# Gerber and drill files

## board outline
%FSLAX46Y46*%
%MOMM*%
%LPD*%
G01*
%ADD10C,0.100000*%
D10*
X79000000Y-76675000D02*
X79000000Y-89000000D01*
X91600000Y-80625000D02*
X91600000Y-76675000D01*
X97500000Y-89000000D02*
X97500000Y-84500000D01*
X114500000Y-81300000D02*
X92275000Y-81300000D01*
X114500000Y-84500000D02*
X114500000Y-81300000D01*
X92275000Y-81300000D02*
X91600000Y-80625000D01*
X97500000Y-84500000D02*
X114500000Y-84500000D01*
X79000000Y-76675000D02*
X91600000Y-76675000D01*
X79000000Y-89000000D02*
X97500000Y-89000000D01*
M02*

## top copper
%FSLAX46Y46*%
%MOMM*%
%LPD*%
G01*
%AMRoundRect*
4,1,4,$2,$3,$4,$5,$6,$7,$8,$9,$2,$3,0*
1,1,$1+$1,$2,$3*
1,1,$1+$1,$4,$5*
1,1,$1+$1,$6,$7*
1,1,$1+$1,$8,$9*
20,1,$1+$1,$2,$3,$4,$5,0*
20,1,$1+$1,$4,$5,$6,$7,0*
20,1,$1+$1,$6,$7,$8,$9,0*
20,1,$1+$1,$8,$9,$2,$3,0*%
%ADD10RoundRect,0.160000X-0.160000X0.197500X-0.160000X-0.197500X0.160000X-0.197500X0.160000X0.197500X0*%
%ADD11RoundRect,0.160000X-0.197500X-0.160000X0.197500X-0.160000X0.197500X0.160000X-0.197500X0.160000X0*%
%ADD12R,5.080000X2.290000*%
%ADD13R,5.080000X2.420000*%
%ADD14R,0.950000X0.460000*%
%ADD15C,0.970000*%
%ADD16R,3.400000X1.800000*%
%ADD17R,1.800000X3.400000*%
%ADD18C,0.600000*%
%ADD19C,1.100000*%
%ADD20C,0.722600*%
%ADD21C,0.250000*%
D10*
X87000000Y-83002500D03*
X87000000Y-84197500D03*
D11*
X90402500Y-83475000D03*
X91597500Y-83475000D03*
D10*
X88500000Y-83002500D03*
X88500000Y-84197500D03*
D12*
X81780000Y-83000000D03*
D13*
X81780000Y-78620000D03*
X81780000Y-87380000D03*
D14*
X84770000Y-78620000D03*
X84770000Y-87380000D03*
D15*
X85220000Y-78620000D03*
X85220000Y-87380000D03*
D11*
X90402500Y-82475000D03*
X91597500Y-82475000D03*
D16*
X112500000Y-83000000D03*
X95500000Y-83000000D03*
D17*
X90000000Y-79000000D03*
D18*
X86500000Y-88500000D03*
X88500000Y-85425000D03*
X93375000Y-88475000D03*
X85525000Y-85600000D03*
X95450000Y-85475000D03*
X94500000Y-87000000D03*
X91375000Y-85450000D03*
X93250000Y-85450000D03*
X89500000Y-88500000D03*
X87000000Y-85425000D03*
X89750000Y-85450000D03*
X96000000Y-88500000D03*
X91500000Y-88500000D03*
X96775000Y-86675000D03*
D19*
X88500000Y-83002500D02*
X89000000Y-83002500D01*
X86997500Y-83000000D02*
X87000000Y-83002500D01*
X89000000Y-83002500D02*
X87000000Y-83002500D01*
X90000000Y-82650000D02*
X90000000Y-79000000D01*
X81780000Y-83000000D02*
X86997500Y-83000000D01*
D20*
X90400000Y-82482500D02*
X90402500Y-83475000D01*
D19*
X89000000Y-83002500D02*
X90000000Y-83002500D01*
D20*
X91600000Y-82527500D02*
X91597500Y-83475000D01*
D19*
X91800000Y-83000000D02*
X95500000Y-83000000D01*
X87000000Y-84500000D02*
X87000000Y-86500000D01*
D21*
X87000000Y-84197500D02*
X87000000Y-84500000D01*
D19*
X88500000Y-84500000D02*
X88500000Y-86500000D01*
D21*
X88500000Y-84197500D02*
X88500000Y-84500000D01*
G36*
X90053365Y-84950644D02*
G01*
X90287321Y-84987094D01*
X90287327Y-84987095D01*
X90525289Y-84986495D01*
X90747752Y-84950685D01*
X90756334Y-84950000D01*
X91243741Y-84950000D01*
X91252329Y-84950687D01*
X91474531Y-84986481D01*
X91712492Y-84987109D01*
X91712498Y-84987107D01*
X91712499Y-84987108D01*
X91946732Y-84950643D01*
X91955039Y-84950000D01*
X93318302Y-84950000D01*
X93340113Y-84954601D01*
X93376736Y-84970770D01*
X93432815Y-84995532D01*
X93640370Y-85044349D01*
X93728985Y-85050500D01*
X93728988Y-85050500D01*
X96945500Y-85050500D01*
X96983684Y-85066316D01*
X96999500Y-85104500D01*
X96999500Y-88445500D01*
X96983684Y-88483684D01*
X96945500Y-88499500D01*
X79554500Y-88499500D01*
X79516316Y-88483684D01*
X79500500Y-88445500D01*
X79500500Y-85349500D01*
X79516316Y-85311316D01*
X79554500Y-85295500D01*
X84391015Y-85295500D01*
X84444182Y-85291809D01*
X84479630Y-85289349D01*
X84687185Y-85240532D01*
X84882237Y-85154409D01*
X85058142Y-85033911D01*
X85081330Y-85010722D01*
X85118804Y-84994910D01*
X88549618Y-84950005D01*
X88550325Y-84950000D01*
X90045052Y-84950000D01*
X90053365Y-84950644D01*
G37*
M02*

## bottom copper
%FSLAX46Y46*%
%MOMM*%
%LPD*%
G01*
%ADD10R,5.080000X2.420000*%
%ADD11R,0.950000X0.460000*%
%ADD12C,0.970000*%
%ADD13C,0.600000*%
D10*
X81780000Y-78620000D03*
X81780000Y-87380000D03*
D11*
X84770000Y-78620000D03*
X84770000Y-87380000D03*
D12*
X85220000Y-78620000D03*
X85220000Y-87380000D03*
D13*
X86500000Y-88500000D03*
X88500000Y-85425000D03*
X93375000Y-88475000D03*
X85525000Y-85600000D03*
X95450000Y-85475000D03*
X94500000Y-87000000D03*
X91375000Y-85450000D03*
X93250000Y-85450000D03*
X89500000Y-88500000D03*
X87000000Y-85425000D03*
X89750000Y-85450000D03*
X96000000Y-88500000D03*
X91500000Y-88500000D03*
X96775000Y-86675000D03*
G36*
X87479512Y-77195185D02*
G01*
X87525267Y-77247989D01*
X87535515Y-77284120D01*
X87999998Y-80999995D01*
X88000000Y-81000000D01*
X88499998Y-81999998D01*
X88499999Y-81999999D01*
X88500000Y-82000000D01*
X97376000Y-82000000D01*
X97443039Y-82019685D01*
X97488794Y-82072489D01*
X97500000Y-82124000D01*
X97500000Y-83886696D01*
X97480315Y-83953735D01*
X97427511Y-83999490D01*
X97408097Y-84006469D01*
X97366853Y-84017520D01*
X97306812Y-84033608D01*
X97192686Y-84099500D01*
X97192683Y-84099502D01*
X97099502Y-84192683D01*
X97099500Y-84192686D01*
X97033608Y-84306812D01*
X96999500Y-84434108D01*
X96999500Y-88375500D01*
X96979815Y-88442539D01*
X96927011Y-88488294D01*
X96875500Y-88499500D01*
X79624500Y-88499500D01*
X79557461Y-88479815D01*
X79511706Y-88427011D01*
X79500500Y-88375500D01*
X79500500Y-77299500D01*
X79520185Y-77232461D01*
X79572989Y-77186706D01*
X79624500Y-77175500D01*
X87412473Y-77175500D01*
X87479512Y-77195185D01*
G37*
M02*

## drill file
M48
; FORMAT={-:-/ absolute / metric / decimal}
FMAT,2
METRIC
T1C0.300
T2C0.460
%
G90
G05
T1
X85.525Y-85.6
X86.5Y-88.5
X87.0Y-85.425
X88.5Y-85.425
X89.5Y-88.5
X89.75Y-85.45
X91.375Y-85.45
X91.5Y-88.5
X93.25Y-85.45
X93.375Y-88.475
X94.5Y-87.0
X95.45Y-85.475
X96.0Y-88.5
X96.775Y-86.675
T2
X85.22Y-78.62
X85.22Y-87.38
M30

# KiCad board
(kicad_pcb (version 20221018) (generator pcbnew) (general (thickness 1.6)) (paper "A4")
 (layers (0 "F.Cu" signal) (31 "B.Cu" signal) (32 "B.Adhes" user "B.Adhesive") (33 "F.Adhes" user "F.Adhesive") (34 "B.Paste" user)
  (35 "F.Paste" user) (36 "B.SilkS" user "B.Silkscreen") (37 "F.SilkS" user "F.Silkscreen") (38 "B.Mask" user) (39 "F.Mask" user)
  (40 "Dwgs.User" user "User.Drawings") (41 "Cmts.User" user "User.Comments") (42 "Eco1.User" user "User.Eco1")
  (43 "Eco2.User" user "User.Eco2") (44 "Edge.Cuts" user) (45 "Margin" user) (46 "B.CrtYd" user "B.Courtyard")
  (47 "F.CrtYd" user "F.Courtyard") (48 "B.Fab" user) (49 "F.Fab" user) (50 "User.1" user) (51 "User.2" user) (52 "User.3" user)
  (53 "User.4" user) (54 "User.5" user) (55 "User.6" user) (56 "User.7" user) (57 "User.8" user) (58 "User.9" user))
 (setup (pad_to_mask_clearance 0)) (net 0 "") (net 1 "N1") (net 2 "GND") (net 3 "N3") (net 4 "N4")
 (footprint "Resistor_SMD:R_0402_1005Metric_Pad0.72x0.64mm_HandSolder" (layer "F.Cu") (at 87 83.6 -90)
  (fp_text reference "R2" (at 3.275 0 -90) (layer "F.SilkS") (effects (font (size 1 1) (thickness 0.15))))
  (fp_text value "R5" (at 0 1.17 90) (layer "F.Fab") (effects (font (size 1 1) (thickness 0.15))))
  (pad "1" smd roundrect (at -0.5975 0 270) (size 0.715 0.64) (layers "F.Cu" "F.Paste" "F.Mask") (roundrect_rratio 0.25) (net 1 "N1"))
  (pad "2" smd roundrect (at 0.5975 0 270) (size 0.715 0.64) (layers "F.Cu" "F.Paste" "F.Mask") (roundrect_rratio 0.25) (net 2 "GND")))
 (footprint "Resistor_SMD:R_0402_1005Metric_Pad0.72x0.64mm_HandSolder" (layer "F.Cu") (at 91 83.475)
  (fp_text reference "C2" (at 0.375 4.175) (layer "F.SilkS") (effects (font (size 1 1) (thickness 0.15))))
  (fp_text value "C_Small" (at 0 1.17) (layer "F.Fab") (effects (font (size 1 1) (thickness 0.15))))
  (pad "1" smd roundrect (at -0.5975 0) (size 0.715 0.64) (layers "F.Cu" "F.Paste" "F.Mask") (roundrect_rratio 0.25) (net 1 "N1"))
  (pad "2" smd roundrect (at 0.5975 0) (size 0.715 0.64) (layers "F.Cu" "F.Paste" "F.Mask") (roundrect_rratio 0.25) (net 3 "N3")))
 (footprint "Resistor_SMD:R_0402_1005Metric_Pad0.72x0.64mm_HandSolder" (layer "F.Cu") (at 88.5 83.6 -90)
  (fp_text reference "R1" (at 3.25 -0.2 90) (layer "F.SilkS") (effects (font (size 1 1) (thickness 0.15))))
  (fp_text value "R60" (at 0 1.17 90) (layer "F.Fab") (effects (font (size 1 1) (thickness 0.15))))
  (pad "1" smd roundrect (at -0.5975 0 270) (size 0.715 0.64) (layers "F.Cu" "F.Paste" "F.Mask") (roundrect_rratio 0.25) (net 1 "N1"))
  (pad "2" smd roundrect (at 0.5975 0 270) (size 0.715 0.64) (layers "F.Cu" "F.Paste" "F.Mask") (roundrect_rratio 0.25) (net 2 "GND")))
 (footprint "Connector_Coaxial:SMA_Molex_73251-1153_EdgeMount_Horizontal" (layer "F.Cu") (at 83.5 83)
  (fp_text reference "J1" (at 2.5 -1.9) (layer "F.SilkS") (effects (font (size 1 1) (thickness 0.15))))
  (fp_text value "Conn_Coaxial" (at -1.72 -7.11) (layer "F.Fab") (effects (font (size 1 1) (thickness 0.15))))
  (pad "1" smd rect (at -1.72 0) (size 5.08 2.29) (layers "F.Cu" "F.Paste" "F.Mask") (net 1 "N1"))
  (pad "2" smd rect (at -1.72 -4.38) (size 5.08 2.42) (layers "F.Cu" "F.Paste" "F.Mask") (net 2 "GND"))
  (pad "2" smd rect (at -1.72 -4.38) (size 5.08 2.42) (layers "B.Cu" "B.Paste" "B.Mask") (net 2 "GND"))
  (pad "2" smd rect (at -1.72 4.38) (size 5.08 2.42) (layers "F.Cu" "F.Paste" "F.Mask") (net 2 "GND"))
  (pad "2" smd rect (at -1.72 4.38) (size 5.08 2.42) (layers "B.Cu" "B.Paste" "B.Mask") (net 2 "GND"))
  (pad "2" smd rect (at 1.27 -4.38) (size 0.95 0.46) (layers "F.Cu") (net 2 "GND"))
  (pad "2" smd rect (at 1.27 -4.38) (size 0.95 0.46) (layers "B.Cu") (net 2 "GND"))
  (pad "2" smd rect (at 1.27 4.38) (size 0.95 0.46) (layers "F.Cu") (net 2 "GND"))
  (pad "2" smd rect (at 1.27 4.38) (size 0.95 0.46) (layers "B.Cu") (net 2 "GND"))
  (pad "2" thru_hole circle (at 1.72 -4.38) (size 0.97 0.97) (drill 0.46) (layers "*.Cu") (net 2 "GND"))
  (pad "2" thru_hole circle (at 1.72 4.38) (size 0.97 0.97) (drill 0.46) (layers "*.Cu") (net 2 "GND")))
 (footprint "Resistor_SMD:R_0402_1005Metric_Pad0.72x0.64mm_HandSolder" (layer "F.Cu") (at 91 82.475)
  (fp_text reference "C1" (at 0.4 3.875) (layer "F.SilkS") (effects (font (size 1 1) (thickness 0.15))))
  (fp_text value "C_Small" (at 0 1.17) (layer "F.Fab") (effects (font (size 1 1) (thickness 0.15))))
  (pad "1" smd roundrect (at -0.5975 0) (size 0.715 0.64) (layers "F.Cu" "F.Paste" "F.Mask") (roundrect_rratio 0.25) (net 1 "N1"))
  (pad "2" smd roundrect (at 0.5975 0) (size 0.715 0.64) (layers "F.Cu" "F.Paste" "F.Mask") (roundrect_rratio 0.25) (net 3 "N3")))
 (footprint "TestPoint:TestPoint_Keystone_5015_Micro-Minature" (layer "F.Cu") (at 112.5 83)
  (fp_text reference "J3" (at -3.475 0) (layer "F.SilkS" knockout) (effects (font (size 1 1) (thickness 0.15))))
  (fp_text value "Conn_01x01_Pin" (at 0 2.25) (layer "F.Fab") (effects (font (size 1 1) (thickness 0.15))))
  (pad "1" smd rect (at 0 0) (size 3.4 1.8) (layers "F.Cu" "F.Paste" "F.Mask") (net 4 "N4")))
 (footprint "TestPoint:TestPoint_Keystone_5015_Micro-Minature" (layer "F.Cu") (at 95.5 83)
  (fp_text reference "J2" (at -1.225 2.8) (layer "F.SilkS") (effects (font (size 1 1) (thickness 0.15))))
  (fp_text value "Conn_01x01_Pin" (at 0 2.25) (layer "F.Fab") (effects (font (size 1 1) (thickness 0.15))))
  (pad "1" smd rect (at 0 0) (size 3.4 1.8) (layers "F.Cu" "F.Paste" "F.Mask") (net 3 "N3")))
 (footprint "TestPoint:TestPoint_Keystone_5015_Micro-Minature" (layer "F.Cu") (at 90 79 90)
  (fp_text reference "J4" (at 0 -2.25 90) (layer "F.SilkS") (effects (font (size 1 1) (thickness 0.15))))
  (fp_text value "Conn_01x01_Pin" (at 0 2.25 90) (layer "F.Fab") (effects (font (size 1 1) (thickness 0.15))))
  (pad "1" smd rect (at 0 0 90) (size 3.4 1.8) (layers "F.Cu" "F.Paste" "F.Mask") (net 1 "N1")))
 (gr_line (start 79 76.675) (end 79 89) (stroke (width 0.1) (type default)) (layer "Edge.Cuts"))
 (gr_line (start 91.6 80.625) (end 91.6 76.675) (stroke (width 0.1) (type default)) (layer "Edge.Cuts"))
 (gr_line (start 97.5 89) (end 97.5 84.5) (stroke (width 0.1) (type default)) (layer "Edge.Cuts"))
 (gr_line (start 114.5 81.3) (end 92.275 81.3) (stroke (width 0.1) (type default)) (layer "Edge.Cuts"))
 (gr_line (start 114.5 84.5) (end 114.5 81.3) (stroke (width 0.1) (type default)) (layer "Edge.Cuts"))
 (gr_line (start 92.275 81.3) (end 91.6 80.625) (stroke (width 0.1) (type default)) (layer "Edge.Cuts"))
 (gr_line (start 97.5 84.5) (end 114.5 84.5) (stroke (width 0.1) (type default)) (layer "Edge.Cuts"))
 (gr_line (start 79 76.675) (end 91.6 76.675) (stroke (width 0.1) (type default)) (layer "Edge.Cuts"))
 (gr_line (start 79 89) (end 97.5 89) (stroke (width 0.1) (type default)) (layer "Edge.Cuts"))
 (segment (start 88.5 83.0025) (end 89 83.0025) (width 1.1) (layer "F.Cu") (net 1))
 (segment (start 86.9975 83) (end 87 83.0025) (width 1.1) (layer "F.Cu") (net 1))
 (segment (start 89 83.0025) (end 87 83.0025) (width 1.1) (layer "F.Cu") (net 1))
 (segment (start 90 82.65) (end 90 79) (width 1.1) (layer "F.Cu") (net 1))
 (segment (start 81.78 83) (end 86.9975 83) (width 1.1) (layer "F.Cu") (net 1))
 (segment (start 90.4 82.4825) (end 90.4025 83.475) (width 0.7226) (layer "F.Cu") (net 1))
 (segment (start 89 83.0025) (end 90 83.0025) (width 1.1) (layer "F.Cu") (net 1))
 (segment (start 91.6 82.5275) (end 91.5975 83.475) (width 0.7226) (layer "F.Cu") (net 3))
 (segment (start 91.8 83) (end 95.5 83) (width 1.1) (layer "F.Cu") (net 3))
 (segment (start 87 84.5) (end 87 86.5) (width 1.1) (layer "F.Cu") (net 2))
 (segment (start 87 84.1975) (end 87 84.5) (width 0.25) (layer "F.Cu") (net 2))
 (segment (start 88.5 84.5) (end 88.5 86.5) (width 1.1) (layer "F.Cu") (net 2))
 (segment (start 88.5 84.1975) (end 88.5 84.5) (width 0.25) (layer "F.Cu") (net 2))
 (via (at 86.5 88.5) (size 0.6) (drill 0.3) (layers "F.Cu" "B.Cu") (free) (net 2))
 (via (at 88.5 85.425) (size 0.6) (drill 0.3) (layers "F.Cu" "B.Cu") (free) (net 2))
 (via (at 93.375 88.475) (size 0.6) (drill 0.3) (layers "F.Cu" "B.Cu") (free) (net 2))
 (via (at 85.525 85.6) (size 0.6) (drill 0.3) (layers "F.Cu" "B.Cu") (free) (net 2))
 (via (at 95.45 85.475) (size 0.6) (drill 0.3) (layers "F.Cu" "B.Cu") (free) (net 2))
 (via (at 94.5 87) (size 0.6) (drill 0.3) (layers "F.Cu" "B.Cu") (free) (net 2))
 (via (at 91.375 85.45) (size 0.6) (drill 0.3) (layers "F.Cu" "B.Cu") (free) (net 2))
 (via (at 93.25 85.45) (size 0.6) (drill 0.3) (layers "F.Cu" "B.Cu") (free) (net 2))
 (via (at 89.5 88.5) (size 0.6) (drill 0.3) (layers "F.Cu" "B.Cu") (free) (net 2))
 (via (at 87 85.425) (size 0.6) (drill 0.3) (layers "F.Cu" "B.Cu") (free) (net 2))
 (via (at 89.75 85.45) (size 0.6) (drill 0.3) (layers "F.Cu" "B.Cu") (free) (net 2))
 (via (at 96 88.5) (size 0.6) (drill 0.3) (layers "F.Cu" "B.Cu") (free) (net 2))
 (via (at 91.5 88.5) (size 0.6) (drill 0.3) (layers "F.Cu" "B.Cu") (free) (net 2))
 (via (at 96.775 86.675) (size 0.6) (drill 0.3) (layers "F.Cu" "B.Cu") (free) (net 2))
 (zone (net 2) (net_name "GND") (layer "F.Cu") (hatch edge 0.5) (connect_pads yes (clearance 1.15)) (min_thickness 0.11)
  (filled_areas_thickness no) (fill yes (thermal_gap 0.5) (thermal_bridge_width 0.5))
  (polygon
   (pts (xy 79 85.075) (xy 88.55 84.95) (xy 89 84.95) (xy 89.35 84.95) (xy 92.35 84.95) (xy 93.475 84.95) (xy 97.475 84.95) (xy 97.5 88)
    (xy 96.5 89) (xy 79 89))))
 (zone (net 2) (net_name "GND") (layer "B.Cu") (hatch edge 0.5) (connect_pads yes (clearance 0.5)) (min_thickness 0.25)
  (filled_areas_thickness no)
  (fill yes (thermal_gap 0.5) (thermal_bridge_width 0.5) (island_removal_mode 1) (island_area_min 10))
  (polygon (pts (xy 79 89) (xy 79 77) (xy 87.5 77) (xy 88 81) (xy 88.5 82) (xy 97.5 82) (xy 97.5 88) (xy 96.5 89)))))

